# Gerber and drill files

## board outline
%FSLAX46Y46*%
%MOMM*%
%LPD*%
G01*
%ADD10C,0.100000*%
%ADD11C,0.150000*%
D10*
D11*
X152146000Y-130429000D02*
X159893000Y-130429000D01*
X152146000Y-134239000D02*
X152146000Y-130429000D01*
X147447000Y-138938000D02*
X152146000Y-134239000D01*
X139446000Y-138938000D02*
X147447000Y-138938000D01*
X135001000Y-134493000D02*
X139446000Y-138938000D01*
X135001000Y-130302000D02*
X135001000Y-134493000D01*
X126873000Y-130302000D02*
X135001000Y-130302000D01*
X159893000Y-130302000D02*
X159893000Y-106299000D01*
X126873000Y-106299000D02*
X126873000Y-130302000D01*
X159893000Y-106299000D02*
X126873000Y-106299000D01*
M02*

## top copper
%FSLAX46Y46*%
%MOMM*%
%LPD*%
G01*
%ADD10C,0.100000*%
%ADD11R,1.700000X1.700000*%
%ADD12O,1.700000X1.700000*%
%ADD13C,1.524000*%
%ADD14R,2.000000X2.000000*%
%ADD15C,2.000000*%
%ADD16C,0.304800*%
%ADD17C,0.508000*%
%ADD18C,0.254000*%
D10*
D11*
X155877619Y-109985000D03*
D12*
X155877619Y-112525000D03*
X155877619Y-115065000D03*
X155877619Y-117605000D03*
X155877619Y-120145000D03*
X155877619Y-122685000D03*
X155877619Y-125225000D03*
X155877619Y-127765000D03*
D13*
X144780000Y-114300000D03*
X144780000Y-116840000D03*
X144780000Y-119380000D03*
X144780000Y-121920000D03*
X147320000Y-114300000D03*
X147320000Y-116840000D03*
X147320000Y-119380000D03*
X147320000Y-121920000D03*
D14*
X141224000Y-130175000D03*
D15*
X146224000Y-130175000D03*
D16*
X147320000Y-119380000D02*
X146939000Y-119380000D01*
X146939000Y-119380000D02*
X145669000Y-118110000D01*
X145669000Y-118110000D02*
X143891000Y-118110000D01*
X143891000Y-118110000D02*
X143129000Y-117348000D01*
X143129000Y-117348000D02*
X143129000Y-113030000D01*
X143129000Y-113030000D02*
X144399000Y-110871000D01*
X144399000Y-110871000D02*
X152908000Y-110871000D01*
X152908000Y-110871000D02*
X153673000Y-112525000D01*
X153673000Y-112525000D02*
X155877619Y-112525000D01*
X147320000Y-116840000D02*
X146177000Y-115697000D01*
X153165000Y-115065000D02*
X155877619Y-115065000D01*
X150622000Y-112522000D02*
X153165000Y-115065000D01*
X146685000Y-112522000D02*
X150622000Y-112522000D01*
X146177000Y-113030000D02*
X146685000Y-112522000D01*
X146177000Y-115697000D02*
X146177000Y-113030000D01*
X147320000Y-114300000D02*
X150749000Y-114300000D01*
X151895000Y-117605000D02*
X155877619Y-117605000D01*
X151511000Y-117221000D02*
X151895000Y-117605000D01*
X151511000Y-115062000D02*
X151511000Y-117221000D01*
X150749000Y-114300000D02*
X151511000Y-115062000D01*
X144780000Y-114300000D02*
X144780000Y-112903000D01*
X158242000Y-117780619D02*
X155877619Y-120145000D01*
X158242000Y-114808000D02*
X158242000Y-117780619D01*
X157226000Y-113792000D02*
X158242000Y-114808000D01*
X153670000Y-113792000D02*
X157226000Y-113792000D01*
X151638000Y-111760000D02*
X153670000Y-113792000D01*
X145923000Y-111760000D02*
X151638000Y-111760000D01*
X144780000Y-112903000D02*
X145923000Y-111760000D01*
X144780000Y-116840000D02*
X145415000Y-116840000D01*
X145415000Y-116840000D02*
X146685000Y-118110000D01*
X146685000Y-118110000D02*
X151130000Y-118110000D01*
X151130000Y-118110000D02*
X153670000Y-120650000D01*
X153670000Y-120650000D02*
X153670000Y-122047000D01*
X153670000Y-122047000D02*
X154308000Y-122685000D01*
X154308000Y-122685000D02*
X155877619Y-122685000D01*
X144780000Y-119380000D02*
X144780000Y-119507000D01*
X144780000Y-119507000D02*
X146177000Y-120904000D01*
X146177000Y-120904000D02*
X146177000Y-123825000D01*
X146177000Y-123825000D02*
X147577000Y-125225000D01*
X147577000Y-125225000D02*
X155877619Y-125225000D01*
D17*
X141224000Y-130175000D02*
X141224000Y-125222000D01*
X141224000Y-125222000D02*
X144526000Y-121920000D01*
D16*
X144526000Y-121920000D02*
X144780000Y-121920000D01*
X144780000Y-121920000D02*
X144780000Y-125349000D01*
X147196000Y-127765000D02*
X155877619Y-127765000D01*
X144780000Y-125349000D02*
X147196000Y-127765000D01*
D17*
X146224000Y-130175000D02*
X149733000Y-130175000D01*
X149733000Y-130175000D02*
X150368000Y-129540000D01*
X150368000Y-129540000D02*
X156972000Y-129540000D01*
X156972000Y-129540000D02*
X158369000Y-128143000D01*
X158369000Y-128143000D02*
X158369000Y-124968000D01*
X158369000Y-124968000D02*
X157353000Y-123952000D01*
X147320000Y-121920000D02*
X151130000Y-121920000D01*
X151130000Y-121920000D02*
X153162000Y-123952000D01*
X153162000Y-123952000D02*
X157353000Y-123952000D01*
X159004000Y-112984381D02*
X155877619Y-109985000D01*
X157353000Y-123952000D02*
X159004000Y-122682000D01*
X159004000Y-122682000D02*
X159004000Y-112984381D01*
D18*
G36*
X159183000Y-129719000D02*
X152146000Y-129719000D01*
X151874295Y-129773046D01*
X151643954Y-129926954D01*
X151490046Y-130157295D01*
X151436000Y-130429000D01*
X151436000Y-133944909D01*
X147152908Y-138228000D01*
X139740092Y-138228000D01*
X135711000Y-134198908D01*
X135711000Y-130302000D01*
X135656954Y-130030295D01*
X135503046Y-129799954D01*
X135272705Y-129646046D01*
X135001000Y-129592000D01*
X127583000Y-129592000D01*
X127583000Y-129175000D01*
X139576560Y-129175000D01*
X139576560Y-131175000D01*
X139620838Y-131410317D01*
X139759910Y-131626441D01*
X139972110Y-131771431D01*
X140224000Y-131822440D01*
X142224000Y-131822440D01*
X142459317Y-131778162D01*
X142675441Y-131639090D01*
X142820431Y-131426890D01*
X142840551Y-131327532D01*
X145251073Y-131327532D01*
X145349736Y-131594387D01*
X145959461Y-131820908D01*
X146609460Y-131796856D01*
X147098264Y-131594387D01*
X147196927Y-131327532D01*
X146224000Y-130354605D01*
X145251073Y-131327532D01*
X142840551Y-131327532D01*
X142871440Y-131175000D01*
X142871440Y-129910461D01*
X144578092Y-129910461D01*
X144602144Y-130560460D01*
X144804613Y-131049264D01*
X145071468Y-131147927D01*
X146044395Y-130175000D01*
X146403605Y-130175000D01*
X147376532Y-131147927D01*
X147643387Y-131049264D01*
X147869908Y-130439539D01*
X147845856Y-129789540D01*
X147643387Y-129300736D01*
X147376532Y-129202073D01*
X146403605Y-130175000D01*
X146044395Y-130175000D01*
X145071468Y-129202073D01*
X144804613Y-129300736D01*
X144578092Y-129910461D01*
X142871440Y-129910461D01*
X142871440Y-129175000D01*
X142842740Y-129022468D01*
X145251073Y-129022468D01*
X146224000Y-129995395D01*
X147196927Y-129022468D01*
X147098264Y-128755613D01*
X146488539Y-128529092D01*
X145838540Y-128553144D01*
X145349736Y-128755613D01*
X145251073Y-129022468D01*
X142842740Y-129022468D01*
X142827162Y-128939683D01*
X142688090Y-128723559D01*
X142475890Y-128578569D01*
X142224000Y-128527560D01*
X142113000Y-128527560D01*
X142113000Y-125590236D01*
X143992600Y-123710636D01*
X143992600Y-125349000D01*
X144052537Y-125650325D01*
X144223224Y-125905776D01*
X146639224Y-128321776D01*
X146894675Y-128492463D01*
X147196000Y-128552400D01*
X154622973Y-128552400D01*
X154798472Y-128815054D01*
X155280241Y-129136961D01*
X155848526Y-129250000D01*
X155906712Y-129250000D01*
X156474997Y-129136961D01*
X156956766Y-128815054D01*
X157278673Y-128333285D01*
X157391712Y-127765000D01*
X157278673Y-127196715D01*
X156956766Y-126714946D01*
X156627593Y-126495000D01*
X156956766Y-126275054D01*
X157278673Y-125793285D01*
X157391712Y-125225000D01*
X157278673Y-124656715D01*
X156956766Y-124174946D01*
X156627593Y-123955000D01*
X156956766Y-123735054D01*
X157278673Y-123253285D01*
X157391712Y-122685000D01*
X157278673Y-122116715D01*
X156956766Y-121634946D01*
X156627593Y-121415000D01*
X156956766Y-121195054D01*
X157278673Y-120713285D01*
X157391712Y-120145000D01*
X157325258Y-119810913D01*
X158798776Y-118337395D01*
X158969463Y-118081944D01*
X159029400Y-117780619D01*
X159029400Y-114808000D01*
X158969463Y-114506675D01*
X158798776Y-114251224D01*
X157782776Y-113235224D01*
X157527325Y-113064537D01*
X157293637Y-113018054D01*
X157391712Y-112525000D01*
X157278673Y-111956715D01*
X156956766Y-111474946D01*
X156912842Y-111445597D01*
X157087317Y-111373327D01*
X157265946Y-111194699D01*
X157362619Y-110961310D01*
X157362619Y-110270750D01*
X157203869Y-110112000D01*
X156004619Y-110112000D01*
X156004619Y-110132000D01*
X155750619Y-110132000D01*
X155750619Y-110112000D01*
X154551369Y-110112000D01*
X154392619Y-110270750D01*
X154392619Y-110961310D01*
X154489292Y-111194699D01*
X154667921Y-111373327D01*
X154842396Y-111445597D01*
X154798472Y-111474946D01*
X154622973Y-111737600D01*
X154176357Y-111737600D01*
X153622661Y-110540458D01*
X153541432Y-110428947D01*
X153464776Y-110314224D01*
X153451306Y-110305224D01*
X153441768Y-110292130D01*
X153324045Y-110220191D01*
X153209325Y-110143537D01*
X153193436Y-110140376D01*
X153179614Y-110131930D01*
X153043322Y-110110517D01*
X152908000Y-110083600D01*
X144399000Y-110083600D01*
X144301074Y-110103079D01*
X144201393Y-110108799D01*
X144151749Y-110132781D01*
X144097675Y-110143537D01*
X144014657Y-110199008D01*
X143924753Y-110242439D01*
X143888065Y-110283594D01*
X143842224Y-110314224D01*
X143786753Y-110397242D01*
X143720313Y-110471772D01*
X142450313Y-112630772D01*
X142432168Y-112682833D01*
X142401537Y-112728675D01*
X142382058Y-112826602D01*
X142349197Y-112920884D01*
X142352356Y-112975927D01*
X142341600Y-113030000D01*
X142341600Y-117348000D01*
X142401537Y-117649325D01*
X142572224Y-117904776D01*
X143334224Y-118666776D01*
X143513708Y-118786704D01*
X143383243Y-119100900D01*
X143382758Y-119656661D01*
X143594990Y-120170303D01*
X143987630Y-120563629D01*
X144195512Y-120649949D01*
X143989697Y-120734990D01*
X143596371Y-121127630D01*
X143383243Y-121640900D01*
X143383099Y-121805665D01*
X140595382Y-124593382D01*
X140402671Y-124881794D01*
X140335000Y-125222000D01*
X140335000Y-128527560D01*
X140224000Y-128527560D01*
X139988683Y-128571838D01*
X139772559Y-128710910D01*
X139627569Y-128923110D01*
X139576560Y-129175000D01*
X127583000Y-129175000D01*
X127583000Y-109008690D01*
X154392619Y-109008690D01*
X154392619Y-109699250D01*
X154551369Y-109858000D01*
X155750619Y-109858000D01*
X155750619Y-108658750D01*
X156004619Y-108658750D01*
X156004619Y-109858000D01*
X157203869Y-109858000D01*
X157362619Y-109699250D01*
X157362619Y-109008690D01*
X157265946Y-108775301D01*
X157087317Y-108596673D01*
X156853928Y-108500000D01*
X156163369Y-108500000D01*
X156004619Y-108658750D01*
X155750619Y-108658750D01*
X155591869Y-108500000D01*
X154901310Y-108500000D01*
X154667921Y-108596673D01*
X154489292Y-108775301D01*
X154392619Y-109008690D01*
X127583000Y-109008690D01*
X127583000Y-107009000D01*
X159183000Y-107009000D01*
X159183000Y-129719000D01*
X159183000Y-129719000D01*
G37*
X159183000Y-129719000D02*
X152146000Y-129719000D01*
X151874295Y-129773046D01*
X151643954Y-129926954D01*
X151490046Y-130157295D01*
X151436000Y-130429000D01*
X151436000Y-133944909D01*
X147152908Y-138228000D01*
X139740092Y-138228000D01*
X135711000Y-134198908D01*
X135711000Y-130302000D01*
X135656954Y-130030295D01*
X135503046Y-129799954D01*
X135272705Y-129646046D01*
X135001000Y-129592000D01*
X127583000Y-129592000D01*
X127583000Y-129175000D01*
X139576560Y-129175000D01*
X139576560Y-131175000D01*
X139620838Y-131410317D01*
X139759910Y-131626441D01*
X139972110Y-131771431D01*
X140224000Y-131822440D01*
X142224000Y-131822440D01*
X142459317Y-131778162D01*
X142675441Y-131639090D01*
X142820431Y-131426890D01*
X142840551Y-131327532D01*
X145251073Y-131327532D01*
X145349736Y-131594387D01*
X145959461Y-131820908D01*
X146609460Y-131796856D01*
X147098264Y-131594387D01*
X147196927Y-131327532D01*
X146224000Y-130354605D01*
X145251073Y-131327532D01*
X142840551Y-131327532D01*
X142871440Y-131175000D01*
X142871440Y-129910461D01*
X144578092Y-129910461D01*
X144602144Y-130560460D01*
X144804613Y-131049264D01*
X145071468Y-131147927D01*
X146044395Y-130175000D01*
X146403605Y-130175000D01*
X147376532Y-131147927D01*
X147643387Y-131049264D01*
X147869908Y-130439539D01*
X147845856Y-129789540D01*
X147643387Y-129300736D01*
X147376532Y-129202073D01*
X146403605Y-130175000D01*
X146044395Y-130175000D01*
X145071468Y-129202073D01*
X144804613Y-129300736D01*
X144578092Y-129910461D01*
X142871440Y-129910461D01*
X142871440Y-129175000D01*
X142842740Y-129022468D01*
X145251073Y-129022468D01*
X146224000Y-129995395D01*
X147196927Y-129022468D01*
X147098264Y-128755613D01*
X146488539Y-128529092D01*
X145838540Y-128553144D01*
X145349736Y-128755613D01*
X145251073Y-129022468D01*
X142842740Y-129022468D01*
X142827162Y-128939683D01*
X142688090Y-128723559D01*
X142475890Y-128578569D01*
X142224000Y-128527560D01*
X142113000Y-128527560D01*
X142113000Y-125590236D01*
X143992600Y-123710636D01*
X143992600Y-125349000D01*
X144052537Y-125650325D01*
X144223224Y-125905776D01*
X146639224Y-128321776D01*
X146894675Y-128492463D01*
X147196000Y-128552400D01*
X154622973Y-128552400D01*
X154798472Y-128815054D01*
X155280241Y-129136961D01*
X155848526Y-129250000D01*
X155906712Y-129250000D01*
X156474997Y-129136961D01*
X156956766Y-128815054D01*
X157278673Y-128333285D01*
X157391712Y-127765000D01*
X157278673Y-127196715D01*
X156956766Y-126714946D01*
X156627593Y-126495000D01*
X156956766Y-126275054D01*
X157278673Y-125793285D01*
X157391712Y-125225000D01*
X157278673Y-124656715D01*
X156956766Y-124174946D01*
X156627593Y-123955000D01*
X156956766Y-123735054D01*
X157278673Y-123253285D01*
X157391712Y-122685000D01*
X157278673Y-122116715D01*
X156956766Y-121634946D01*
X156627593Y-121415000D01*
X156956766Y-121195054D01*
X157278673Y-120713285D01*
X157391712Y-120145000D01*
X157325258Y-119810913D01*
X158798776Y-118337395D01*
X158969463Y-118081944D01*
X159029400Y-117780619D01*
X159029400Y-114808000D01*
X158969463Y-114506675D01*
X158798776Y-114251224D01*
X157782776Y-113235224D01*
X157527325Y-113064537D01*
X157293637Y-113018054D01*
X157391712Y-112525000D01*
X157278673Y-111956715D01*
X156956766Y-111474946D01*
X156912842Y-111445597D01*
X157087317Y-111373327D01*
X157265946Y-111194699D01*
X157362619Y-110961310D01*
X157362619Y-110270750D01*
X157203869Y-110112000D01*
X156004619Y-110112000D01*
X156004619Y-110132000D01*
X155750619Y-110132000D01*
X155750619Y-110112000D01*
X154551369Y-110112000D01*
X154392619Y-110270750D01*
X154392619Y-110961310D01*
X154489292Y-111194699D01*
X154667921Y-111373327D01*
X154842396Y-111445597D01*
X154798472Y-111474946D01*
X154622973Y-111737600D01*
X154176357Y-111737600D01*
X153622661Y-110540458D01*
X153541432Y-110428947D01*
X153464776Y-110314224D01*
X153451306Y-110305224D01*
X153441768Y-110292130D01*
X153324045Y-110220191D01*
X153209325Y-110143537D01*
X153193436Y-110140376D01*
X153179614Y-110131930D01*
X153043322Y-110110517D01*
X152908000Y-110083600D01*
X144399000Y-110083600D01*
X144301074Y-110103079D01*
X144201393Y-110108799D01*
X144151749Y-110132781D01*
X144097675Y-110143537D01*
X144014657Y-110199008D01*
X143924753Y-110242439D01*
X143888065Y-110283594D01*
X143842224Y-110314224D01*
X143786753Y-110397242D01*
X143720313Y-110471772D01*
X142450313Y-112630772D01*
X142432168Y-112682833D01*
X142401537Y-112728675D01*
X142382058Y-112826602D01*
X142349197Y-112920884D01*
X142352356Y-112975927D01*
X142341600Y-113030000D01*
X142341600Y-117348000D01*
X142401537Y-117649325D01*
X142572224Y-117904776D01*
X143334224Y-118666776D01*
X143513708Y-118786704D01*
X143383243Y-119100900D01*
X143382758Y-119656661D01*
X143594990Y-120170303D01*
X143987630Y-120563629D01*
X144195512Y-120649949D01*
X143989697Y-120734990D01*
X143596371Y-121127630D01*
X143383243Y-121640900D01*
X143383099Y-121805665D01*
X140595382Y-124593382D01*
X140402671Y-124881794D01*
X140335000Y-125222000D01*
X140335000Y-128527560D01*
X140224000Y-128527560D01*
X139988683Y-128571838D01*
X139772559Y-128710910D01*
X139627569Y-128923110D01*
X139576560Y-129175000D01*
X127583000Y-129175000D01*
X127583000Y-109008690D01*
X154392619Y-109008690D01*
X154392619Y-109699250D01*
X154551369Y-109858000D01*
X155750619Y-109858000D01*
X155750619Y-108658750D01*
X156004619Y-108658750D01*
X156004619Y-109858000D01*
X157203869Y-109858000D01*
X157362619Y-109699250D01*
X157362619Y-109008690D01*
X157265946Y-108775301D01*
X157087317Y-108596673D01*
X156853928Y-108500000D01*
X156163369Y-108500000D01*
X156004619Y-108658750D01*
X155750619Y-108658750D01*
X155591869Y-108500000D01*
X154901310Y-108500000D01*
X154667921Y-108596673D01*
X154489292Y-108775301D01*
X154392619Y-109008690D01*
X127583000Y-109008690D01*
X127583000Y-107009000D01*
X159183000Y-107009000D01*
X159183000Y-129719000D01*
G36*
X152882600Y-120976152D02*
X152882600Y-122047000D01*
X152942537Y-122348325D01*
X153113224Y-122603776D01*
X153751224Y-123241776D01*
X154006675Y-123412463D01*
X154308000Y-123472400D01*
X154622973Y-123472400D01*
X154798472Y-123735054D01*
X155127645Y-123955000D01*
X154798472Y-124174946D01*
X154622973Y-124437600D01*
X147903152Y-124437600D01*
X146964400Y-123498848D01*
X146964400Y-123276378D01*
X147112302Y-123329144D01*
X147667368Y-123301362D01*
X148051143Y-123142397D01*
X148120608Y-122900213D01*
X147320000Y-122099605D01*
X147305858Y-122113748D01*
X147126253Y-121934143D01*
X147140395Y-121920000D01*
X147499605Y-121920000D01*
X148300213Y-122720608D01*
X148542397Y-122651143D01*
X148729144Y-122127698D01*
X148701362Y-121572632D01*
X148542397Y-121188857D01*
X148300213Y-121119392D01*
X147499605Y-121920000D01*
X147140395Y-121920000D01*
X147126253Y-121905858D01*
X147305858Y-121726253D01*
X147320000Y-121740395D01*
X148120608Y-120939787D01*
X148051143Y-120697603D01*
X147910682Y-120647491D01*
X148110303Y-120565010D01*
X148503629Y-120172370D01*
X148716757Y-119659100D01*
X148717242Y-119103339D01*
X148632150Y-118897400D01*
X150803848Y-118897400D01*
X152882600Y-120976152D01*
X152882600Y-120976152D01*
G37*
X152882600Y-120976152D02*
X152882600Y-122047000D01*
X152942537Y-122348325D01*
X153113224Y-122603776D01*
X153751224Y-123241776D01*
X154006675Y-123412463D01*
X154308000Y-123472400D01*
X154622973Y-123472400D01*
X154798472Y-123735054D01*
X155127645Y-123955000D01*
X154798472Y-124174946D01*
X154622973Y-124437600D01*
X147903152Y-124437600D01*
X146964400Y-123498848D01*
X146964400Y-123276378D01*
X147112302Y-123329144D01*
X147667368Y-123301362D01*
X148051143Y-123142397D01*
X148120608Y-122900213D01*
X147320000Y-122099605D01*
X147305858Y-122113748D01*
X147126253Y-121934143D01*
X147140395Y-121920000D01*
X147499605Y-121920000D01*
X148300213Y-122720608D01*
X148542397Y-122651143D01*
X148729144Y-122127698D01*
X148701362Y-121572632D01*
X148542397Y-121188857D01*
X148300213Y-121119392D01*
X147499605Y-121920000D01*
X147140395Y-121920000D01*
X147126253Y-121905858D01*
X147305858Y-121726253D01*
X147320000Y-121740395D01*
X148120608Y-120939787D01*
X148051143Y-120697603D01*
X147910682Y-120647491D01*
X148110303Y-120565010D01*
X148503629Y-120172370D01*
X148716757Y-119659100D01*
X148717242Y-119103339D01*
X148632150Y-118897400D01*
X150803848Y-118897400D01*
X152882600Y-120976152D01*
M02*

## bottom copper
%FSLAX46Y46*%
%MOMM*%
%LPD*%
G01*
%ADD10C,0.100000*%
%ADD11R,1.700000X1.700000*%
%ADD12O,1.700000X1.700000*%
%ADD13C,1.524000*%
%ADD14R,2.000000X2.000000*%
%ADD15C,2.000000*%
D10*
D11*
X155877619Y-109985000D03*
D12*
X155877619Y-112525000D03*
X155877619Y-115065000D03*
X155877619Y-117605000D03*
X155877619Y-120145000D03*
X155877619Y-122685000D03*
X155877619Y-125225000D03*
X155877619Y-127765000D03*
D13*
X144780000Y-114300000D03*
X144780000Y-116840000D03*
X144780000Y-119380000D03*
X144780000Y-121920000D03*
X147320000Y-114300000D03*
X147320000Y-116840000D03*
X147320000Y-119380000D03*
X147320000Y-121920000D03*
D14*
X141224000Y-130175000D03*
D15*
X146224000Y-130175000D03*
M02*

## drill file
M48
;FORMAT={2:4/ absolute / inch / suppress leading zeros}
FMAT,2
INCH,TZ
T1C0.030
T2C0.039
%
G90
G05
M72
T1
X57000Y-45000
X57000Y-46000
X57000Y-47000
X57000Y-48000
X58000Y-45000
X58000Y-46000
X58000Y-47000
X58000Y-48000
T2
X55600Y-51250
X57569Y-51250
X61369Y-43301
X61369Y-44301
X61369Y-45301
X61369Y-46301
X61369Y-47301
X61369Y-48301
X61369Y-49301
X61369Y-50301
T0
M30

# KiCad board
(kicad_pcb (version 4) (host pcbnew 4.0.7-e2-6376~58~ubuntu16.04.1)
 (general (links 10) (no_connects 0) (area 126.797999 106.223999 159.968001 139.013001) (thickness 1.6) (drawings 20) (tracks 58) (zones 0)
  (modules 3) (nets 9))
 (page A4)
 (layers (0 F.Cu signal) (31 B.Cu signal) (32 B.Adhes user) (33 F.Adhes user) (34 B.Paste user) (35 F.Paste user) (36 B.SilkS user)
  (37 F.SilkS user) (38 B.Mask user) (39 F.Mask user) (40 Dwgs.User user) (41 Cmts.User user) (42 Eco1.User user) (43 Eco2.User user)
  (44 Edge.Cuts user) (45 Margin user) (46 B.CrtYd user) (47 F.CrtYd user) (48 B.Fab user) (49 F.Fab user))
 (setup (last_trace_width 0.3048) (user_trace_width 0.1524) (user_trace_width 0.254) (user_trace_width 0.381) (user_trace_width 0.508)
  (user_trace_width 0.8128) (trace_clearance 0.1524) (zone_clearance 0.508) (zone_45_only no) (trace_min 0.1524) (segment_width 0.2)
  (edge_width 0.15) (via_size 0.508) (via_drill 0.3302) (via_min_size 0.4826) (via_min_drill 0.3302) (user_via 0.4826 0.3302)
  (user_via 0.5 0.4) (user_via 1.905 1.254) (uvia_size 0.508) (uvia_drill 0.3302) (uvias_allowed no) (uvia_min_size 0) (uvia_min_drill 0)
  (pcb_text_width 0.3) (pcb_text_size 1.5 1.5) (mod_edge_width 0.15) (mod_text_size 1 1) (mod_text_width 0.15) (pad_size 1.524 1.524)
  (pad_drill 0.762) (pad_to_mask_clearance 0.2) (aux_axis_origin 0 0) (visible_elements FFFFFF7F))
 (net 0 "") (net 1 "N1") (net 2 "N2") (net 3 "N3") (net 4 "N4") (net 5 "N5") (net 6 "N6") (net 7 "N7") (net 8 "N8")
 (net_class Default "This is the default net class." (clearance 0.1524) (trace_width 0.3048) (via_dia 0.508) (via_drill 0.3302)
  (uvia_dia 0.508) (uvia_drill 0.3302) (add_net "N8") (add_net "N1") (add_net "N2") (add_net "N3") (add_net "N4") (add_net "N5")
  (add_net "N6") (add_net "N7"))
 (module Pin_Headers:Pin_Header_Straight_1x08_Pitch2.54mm (layer F.Cu) (at 155.877619 109.985)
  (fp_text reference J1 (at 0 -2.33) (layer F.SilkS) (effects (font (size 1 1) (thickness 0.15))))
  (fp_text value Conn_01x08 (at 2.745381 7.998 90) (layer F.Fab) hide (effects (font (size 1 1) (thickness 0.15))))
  (pad 1 thru_hole rect (at 0 0) (size 1.7 1.7) (drill 1) (layers *.Cu *.Mask) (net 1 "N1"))
  (pad 2 thru_hole oval (at 0 2.54) (size 1.7 1.7) (drill 1) (layers *.Cu *.Mask) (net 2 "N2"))
  (pad 3 thru_hole oval (at 0 5.08) (size 1.7 1.7) (drill 1) (layers *.Cu *.Mask) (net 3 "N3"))
  (pad 4 thru_hole oval (at 0 7.62) (size 1.7 1.7) (drill 1) (layers *.Cu *.Mask) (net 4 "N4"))
  (pad 5 thru_hole oval (at 0 10.16) (size 1.7 1.7) (drill 1) (layers *.Cu *.Mask) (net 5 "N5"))
  (pad 6 thru_hole oval (at 0 12.7) (size 1.7 1.7) (drill 1) (layers *.Cu *.Mask) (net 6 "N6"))
  (pad 7 thru_hole oval (at 0 15.24) (size 1.7 1.7) (drill 1) (layers *.Cu *.Mask) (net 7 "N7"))
  (pad 8 thru_hole oval (at 0 17.78) (size 1.7 1.7) (drill 1) (layers *.Cu *.Mask) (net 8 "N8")))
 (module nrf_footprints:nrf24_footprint (layer F.Cu) (at 137.16 119.38)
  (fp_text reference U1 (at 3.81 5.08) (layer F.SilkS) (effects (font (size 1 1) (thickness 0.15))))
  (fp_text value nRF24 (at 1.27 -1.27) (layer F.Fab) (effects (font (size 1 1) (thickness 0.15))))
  (pad 4 thru_hole circle (at 7.62 -5.08) (size 1.524 1.524) (drill 0.762) (layers *.Cu *.Mask) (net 5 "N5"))
  (pad 5 thru_hole circle (at 7.62 -2.54) (size 1.524 1.524) (drill 0.762) (layers *.Cu *.Mask) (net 6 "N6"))
  (pad 6 thru_hole circle (at 7.62 0) (size 1.524 1.524) (drill 0.762) (layers *.Cu *.Mask) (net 7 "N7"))
  (pad 7 thru_hole circle (at 7.62 2.54) (size 1.524 1.524) (drill 0.762) (layers *.Cu *.Mask) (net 8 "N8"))
  (pad 3 thru_hole circle (at 10.16 -5.08) (size 1.524 1.524) (drill 0.762) (layers *.Cu *.Mask) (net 4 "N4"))
  (pad 2 thru_hole circle (at 10.16 -2.54) (size 1.524 1.524) (drill 0.762) (layers *.Cu *.Mask) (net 3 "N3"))
  (pad 1 thru_hole circle (at 10.16 0) (size 1.524 1.524) (drill 0.762) (layers *.Cu *.Mask) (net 2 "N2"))
  (pad 0 thru_hole circle (at 10.16 2.54) (size 1.524 1.524) (drill 0.762) (layers *.Cu *.Mask) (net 1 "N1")))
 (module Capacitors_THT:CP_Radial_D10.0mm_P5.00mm (layer F.Cu) (at 141.224 130.175)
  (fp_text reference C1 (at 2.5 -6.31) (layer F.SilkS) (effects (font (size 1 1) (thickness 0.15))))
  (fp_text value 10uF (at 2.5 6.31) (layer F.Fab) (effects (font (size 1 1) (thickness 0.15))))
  (pad 1 thru_hole rect (at 0 0) (size 2 2) (drill 1) (layers *.Cu *.Mask) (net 8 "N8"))
  (pad 2 thru_hole circle (at 5 0) (size 2 2) (drill 1) (layers *.Cu *.Mask) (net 1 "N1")))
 (gr_line (start 152.146 130.429) (end 159.893 130.429) (angle 90) (layer Edge.Cuts) (width 0.15))
 (gr_line (start 152.146 134.239) (end 152.146 130.429) (angle 90) (layer Edge.Cuts) (width 0.15))
 (gr_line (start 147.447 138.938) (end 152.146 134.239) (angle 90) (layer Edge.Cuts) (width 0.15))
 (gr_line (start 139.446 138.938) (end 147.447 138.938) (angle 90) (layer Edge.Cuts) (width 0.15))
 (gr_line (start 135.001 134.493) (end 139.446 138.938) (angle 90) (layer Edge.Cuts) (width 0.15))
 (gr_line (start 135.001 130.302) (end 135.001 134.493) (angle 90) (layer Edge.Cuts) (width 0.15))
 (gr_line (start 126.873 130.302) (end 135.001 130.302) (angle 90) (layer Edge.Cuts) (width 0.15))
 (gr_line (start 159.893 130.302) (end 159.893 106.299) (angle 90) (layer Edge.Cuts) (width 0.15))
 (gr_line (start 126.873 106.299) (end 126.873 130.302) (angle 90) (layer Edge.Cuts) (width 0.15))
 (gr_line (start 159.893 106.299) (end 126.873 106.299) (angle 90) (layer Edge.Cuts) (width 0.15))
 (segment (start 147.32 119.38) (end 146.939 119.38) (width 0.3048) (layer F.Cu) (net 2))
 (segment (start 146.939 119.38) (end 145.669 118.11) (width 0.3048) (layer F.Cu) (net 2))
 (segment (start 145.669 118.11) (end 143.891 118.11) (width 0.3048) (layer F.Cu) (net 2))
 (segment (start 143.891 118.11) (end 143.129 117.348) (width 0.3048) (layer F.Cu) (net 2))
 (segment (start 143.129 117.348) (end 143.129 113.03) (width 0.3048) (layer F.Cu) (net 2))
 (segment (start 143.129 113.03) (end 144.399 110.871) (width 0.3048) (layer F.Cu) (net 2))
 (segment (start 144.399 110.871) (end 152.908 110.871) (width 0.3048) (layer F.Cu) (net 2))
 (segment (start 152.908 110.871) (end 153.673 112.525) (width 0.3048) (layer F.Cu) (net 2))
 (segment (start 153.673 112.525) (end 155.877619 112.525) (width 0.3048) (layer F.Cu) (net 2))
 (segment (start 147.32 116.84) (end 146.177 115.697) (width 0.3048) (layer F.Cu) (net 3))
 (segment (start 153.165 115.065) (end 155.877619 115.065) (width 0.3048) (layer F.Cu) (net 3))
 (segment (start 150.622 112.522) (end 153.165 115.065) (width 0.3048) (layer F.Cu) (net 3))
 (segment (start 146.685 112.522) (end 150.622 112.522) (width 0.3048) (layer F.Cu) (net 3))
 (segment (start 146.177 113.03) (end 146.685 112.522) (width 0.3048) (layer F.Cu) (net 3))
 (segment (start 146.177 115.697) (end 146.177 113.03) (width 0.3048) (layer F.Cu) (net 3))
 (segment (start 147.32 114.3) (end 150.749 114.3) (width 0.3048) (layer F.Cu) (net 4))
 (segment (start 151.895 117.605) (end 155.877619 117.605) (width 0.3048) (layer F.Cu) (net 4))
 (segment (start 151.511 117.221) (end 151.895 117.605) (width 0.3048) (layer F.Cu) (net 4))
 (segment (start 151.511 115.062) (end 151.511 117.221) (width 0.3048) (layer F.Cu) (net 4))
 (segment (start 150.749 114.3) (end 151.511 115.062) (width 0.3048) (layer F.Cu) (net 4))
 (segment (start 144.78 114.3) (end 144.78 112.903) (width 0.3048) (layer F.Cu) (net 5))
 (segment (start 158.242 117.780619) (end 155.877619 120.145) (width 0.3048) (layer F.Cu) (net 5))
 (segment (start 158.242 114.808) (end 158.242 117.780619) (width 0.3048) (layer F.Cu) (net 5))
 (segment (start 157.226 113.792) (end 158.242 114.808) (width 0.3048) (layer F.Cu) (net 5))
 (segment (start 153.67 113.792) (end 157.226 113.792) (width 0.3048) (layer F.Cu) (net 5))
 (segment (start 151.638 111.76) (end 153.67 113.792) (width 0.3048) (layer F.Cu) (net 5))
 (segment (start 145.923 111.76) (end 151.638 111.76) (width 0.3048) (layer F.Cu) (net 5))
 (segment (start 144.78 112.903) (end 145.923 111.76) (width 0.3048) (layer F.Cu) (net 5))
 (segment (start 144.78 116.84) (end 145.415 116.84) (width 0.3048) (layer F.Cu) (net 6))
 (segment (start 145.415 116.84) (end 146.685 118.11) (width 0.3048) (layer F.Cu) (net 6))
 (segment (start 146.685 118.11) (end 151.13 118.11) (width 0.3048) (layer F.Cu) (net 6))
 (segment (start 151.13 118.11) (end 153.67 120.65) (width 0.3048) (layer F.Cu) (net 6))
 (segment (start 153.67 120.65) (end 153.67 122.047) (width 0.3048) (layer F.Cu) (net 6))
 (segment (start 153.67 122.047) (end 154.308 122.685) (width 0.3048) (layer F.Cu) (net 6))
 (segment (start 154.308 122.685) (end 155.877619 122.685) (width 0.3048) (layer F.Cu) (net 6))
 (segment (start 144.78 119.38) (end 144.78 119.507) (width 0.3048) (layer F.Cu) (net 7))
 (segment (start 144.78 119.507) (end 146.177 120.904) (width 0.3048) (layer F.Cu) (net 7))
 (segment (start 146.177 120.904) (end 146.177 123.825) (width 0.3048) (layer F.Cu) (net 7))
 (segment (start 146.177 123.825) (end 147.577 125.225) (width 0.3048) (layer F.Cu) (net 7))
 (segment (start 147.577 125.225) (end 155.877619 125.225) (width 0.3048) (layer F.Cu) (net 7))
 (segment (start 141.224 130.175) (end 141.224 125.222) (width 0.508) (layer F.Cu) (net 8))
 (segment (start 141.224 125.222) (end 144.526 121.92) (width 0.508) (layer F.Cu) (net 8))
 (segment (start 144.526 121.92) (end 144.78 121.92) (width 0.3048) (layer F.Cu) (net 8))
 (segment (start 144.78 121.92) (end 144.78 125.349) (width 0.3048) (layer F.Cu) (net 8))
 (segment (start 147.196 127.765) (end 155.877619 127.765) (width 0.3048) (layer F.Cu) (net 8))
 (segment (start 144.78 125.349) (end 147.196 127.765) (width 0.3048) (layer F.Cu) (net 8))
 (segment (start 146.224 130.175) (end 149.733 130.175) (width 0.508) (layer F.Cu) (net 1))
 (segment (start 149.733 130.175) (end 150.368 129.54) (width 0.508) (layer F.Cu) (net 1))
 (segment (start 150.368 129.54) (end 156.972 129.54) (width 0.508) (layer F.Cu) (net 1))
 (segment (start 156.972 129.54) (end 158.369 128.143) (width 0.508) (layer F.Cu) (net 1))
 (segment (start 158.369 128.143) (end 158.369 124.968) (width 0.508) (layer F.Cu) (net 1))
 (segment (start 158.369 124.968) (end 157.353 123.952) (width 0.508) (layer F.Cu) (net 1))
 (segment (start 147.32 121.92) (end 151.13 121.92) (width 0.508) (layer F.Cu) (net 1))
 (segment (start 151.13 121.92) (end 153.162 123.952) (width 0.508) (layer F.Cu) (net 1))
 (segment (start 153.162 123.952) (end 157.353 123.952) (width 0.508) (layer F.Cu) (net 1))
 (segment (start 159.004 112.984381) (end 155.877619 109.985) (width 0.508) (layer F.Cu) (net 1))
 (segment (start 157.353 123.952) (end 159.004 122.682) (width 0.508) (layer F.Cu) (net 1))
 (segment (start 159.004 122.682) (end 159.004 112.984381) (width 0.508) (layer F.Cu) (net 1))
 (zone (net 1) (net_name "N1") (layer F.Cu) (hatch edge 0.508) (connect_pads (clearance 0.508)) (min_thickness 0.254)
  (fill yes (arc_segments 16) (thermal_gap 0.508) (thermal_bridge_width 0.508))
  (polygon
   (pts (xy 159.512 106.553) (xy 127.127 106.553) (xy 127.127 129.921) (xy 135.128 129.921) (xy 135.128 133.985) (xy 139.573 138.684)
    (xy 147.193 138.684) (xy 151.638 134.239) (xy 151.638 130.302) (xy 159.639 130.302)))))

